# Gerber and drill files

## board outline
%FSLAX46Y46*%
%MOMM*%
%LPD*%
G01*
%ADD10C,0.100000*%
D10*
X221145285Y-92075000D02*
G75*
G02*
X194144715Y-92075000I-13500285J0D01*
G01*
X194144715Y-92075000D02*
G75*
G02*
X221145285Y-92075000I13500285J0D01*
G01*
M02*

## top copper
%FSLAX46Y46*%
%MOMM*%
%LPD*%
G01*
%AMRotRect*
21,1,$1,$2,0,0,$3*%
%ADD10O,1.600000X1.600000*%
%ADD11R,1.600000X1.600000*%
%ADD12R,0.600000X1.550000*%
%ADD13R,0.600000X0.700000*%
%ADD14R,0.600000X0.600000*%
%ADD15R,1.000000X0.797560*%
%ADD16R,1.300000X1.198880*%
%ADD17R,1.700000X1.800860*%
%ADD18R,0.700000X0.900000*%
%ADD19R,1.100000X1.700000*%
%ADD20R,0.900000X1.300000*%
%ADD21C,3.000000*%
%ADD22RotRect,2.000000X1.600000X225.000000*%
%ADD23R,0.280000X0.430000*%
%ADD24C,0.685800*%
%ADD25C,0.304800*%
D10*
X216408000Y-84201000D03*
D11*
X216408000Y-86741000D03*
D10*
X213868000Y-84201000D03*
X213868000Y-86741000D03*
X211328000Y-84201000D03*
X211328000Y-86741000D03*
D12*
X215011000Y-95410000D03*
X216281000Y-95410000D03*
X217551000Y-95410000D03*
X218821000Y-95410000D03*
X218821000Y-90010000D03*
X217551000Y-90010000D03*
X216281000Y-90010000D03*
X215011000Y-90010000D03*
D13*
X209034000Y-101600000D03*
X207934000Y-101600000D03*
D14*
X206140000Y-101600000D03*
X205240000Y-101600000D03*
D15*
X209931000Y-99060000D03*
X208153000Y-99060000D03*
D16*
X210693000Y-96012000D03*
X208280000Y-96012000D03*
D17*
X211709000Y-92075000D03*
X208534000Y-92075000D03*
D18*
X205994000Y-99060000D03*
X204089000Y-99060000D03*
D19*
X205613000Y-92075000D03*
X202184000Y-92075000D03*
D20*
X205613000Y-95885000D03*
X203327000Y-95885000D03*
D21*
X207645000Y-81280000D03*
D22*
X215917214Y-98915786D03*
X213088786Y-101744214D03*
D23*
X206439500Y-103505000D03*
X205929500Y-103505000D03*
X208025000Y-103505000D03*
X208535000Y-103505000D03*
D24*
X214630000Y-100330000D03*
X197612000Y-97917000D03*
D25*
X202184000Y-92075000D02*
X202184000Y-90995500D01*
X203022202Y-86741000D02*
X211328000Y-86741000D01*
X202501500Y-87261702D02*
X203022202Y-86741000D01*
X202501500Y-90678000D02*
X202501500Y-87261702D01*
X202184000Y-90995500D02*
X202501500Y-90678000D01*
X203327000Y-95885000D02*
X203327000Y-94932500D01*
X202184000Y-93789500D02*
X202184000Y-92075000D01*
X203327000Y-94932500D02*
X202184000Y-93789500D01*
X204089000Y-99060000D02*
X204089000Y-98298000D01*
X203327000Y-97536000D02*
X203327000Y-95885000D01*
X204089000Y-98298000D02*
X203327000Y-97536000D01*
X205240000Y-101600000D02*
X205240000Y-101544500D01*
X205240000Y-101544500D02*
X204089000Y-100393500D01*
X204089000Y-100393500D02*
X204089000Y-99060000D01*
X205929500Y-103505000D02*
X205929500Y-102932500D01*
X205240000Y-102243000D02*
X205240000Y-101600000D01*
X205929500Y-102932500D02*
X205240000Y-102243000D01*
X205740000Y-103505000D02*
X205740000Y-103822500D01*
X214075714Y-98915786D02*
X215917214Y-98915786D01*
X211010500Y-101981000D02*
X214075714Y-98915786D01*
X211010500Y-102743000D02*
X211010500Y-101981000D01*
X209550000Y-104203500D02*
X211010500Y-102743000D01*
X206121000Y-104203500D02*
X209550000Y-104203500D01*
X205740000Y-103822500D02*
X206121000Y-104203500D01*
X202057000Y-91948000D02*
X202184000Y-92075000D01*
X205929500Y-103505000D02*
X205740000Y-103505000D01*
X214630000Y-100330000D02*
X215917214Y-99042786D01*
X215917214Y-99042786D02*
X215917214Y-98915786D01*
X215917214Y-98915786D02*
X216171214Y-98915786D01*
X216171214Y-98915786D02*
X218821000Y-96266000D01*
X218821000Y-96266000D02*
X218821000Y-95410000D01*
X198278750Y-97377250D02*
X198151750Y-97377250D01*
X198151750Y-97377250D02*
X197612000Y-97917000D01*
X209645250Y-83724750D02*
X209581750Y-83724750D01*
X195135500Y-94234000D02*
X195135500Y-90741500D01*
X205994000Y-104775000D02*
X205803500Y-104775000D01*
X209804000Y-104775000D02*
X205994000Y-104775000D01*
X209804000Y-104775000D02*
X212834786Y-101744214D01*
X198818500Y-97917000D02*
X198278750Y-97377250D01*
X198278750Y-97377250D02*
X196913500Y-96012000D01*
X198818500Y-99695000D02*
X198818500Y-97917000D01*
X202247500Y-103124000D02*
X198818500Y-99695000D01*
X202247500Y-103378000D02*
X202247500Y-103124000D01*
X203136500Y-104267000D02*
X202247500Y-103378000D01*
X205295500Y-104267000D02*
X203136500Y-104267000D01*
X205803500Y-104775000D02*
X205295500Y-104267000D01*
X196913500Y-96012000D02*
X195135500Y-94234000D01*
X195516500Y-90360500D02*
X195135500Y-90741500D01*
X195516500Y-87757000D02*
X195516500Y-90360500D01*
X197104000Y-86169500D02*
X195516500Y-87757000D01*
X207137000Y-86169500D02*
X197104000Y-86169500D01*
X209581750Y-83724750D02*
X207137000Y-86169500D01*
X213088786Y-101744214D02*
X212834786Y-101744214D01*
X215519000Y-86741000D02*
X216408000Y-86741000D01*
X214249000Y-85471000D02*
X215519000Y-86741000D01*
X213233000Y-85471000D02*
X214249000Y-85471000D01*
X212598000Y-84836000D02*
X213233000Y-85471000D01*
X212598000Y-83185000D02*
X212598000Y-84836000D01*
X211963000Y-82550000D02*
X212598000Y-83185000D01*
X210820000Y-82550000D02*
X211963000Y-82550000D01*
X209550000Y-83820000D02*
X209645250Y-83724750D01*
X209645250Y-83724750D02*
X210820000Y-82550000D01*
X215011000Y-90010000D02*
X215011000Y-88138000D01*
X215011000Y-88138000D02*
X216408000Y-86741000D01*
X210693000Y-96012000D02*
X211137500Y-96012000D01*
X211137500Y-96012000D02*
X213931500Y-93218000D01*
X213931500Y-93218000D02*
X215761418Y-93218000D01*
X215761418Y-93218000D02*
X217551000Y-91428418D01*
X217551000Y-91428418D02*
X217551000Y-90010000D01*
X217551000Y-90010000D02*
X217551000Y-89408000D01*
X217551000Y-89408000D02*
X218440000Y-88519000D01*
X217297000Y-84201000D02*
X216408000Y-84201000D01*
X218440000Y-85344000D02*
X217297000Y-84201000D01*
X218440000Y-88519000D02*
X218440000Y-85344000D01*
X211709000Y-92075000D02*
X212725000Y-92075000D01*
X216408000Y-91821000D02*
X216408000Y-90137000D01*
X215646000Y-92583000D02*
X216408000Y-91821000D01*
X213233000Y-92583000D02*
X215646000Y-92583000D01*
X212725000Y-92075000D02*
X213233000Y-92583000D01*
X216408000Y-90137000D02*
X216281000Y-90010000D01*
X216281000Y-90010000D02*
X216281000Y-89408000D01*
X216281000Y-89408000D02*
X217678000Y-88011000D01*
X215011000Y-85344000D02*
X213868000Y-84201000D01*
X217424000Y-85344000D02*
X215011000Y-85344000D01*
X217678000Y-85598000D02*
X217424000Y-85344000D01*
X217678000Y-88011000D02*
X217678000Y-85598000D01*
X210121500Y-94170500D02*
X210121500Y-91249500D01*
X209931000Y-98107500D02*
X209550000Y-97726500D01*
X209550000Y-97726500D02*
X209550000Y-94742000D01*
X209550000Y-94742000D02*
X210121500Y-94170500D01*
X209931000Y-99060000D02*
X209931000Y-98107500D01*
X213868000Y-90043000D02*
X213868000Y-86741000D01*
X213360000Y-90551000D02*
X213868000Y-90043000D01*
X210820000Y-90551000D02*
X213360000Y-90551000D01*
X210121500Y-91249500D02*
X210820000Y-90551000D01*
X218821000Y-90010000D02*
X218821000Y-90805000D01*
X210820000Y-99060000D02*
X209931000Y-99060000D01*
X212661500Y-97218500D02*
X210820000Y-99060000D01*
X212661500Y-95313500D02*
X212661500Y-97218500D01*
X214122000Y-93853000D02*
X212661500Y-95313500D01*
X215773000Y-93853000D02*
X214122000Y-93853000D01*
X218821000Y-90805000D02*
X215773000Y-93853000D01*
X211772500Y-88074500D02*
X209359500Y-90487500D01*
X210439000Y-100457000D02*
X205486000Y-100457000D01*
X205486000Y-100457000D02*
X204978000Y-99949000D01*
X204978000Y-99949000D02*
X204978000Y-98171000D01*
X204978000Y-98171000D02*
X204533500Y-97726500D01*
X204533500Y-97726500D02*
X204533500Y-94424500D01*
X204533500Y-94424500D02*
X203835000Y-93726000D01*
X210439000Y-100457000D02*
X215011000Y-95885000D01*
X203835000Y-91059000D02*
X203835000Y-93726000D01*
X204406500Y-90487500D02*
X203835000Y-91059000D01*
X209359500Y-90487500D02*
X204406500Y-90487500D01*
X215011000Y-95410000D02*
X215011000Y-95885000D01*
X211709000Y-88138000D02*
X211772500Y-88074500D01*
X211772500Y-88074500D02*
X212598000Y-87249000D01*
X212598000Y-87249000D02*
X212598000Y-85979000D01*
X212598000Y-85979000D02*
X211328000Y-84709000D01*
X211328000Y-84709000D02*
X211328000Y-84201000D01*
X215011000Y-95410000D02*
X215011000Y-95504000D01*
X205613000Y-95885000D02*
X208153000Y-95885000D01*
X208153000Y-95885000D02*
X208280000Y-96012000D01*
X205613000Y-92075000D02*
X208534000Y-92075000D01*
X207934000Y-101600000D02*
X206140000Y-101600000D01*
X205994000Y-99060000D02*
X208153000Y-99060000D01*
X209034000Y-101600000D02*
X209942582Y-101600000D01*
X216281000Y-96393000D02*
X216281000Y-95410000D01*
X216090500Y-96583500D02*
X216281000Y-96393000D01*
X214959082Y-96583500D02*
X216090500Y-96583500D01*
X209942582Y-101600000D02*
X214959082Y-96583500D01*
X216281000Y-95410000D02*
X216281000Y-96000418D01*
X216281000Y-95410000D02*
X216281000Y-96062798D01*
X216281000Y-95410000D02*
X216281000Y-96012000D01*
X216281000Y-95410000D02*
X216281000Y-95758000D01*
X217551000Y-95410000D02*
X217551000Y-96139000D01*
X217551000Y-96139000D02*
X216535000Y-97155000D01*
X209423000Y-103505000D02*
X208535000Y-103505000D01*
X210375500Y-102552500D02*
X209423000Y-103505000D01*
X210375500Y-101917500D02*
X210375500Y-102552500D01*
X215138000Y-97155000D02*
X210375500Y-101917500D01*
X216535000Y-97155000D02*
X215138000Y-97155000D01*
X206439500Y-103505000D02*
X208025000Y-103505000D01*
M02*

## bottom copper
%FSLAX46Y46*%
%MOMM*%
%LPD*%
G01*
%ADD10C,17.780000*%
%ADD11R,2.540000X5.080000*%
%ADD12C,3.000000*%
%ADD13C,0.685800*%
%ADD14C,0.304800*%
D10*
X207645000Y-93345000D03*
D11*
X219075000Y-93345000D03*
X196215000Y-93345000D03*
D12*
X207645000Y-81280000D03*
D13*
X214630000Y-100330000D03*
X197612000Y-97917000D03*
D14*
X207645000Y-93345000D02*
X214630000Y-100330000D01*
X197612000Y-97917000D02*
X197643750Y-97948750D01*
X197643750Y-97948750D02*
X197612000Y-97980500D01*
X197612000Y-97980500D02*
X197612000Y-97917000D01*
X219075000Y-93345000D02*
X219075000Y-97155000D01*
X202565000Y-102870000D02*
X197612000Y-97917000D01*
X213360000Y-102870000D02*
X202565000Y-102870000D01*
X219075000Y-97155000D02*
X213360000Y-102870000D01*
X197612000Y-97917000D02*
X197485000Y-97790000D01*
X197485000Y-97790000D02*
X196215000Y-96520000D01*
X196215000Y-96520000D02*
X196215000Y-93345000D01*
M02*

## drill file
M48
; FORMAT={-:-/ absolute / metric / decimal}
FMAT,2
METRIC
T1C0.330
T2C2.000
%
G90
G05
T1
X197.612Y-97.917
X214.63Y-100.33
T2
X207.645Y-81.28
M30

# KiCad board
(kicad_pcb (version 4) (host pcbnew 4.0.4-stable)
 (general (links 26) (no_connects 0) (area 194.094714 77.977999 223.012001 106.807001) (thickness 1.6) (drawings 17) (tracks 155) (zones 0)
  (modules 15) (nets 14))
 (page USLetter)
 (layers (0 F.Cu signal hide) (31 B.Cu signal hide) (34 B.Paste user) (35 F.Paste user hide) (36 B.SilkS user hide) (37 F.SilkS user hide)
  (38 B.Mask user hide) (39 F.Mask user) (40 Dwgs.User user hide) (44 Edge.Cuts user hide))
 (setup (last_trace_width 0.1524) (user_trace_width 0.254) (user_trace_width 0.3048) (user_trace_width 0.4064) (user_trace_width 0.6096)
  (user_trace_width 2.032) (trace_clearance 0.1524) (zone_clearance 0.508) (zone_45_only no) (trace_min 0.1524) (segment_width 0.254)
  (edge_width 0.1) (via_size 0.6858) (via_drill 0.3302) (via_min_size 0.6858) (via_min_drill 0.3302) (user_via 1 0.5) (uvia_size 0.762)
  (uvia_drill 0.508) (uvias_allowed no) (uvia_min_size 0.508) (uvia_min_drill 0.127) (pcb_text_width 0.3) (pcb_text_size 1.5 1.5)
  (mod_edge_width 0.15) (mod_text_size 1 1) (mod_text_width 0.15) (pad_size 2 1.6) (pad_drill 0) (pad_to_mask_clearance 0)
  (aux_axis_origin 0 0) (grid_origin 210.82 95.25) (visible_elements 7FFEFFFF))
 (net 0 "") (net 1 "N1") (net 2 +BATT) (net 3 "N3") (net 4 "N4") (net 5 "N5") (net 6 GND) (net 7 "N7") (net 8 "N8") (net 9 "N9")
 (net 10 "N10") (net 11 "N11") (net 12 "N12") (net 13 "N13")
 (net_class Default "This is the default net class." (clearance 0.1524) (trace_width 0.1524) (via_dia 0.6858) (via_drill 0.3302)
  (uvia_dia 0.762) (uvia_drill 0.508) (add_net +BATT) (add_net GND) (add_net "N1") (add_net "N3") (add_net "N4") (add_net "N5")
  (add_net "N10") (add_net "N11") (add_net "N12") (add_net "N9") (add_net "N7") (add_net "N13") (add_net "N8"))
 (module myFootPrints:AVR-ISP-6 (layer F.Cu) (at 216.408 84.201 270)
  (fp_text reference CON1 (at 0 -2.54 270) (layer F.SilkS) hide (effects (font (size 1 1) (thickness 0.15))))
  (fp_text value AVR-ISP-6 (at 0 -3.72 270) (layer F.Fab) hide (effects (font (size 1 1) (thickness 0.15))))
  (pad 1 smd oval (at 0 0 270) (size 1.6 1.6) (layers F.Cu F.Paste F.Mask) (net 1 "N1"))
  (pad 2 smd rect (at 2.54 0 270) (size 1.6 1.6) (layers F.Cu F.Paste F.Mask) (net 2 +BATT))
  (pad 3 smd oval (at 0 2.54 270) (size 1.6 1.6) (layers F.Cu F.Paste F.Mask) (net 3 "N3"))
  (pad 4 smd oval (at 2.54 2.54 270) (size 1.6 1.6) (layers F.Cu F.Paste F.Mask) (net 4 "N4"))
  (pad 5 smd oval (at 0 5.08 270) (size 1.6 1.6) (layers F.Cu F.Paste F.Mask) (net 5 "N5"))
  (pad 6 smd oval (at 2.54 5.08 270) (size 1.6 1.6) (layers F.Cu F.Paste F.Mask) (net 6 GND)))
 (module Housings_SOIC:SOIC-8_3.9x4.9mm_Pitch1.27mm (layer F.Cu) (at 216.916 92.71 90)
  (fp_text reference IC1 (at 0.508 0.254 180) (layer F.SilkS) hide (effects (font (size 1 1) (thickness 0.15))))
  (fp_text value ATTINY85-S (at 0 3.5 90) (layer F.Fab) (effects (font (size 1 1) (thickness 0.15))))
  (pad 1 smd rect (at -2.7 -1.905 90) (size 1.55 0.6) (layers F.Cu F.Paste F.Mask) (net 5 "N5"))
  (pad 2 smd rect (at -2.7 -0.635 90) (size 1.55 0.6) (layers F.Cu F.Paste F.Mask) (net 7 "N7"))
  (pad 3 smd rect (at -2.7 0.635 90) (size 1.55 0.6) (layers F.Cu F.Paste F.Mask) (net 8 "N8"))
  (pad 4 smd rect (at -2.7 1.905 90) (size 1.55 0.6) (layers F.Cu F.Paste F.Mask) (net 6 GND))
  (pad 5 smd rect (at 2.7 1.905 90) (size 1.55 0.6) (layers F.Cu F.Paste F.Mask) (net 4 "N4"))
  (pad 6 smd rect (at 2.7 0.635 90) (size 1.55 0.6) (layers F.Cu F.Paste F.Mask) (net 1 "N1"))
  (pad 7 smd rect (at 2.7 -0.635 90) (size 1.55 0.6) (layers F.Cu F.Paste F.Mask) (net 3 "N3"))
  (pad 8 smd rect (at 2.7 -1.905 90) (size 1.55 0.6) (layers F.Cu F.Paste F.Mask) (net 2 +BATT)))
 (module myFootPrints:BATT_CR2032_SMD (layer B.Cu) (at 207.645 93.345 180)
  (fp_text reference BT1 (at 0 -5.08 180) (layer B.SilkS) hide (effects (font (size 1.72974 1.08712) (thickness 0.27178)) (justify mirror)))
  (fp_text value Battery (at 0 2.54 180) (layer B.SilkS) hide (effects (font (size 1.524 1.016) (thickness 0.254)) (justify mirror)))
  (pad 2 smd circle (at 0 0 180) (size 17.78 17.78) (layers B.Cu B.Paste B.Mask) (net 6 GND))
  (pad 1 smd rect (at -11.43 0 180) (size 2.54 5.08) (layers B.Cu B.Paste B.Mask) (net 2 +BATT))
  (pad 1 smd rect (at 11.43 0 180) (size 2.54 5.08) (layers B.Cu B.Paste B.Mask) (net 2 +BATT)))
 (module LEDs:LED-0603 (layer F.Cu) (at 208.534 101.6)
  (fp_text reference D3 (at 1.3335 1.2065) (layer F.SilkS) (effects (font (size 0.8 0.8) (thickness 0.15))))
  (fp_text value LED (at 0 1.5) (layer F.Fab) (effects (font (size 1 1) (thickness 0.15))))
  (pad 2 smd rect (at 0.5 0 180) (size 0.6 0.7) (layers F.Cu F.Paste F.Mask) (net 7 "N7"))
  (pad 1 smd rect (at -0.6 0 180) (size 0.6 0.7) (layers F.Cu F.Paste F.Mask) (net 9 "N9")))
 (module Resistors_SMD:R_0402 (layer F.Cu) (at 205.74 101.6 180)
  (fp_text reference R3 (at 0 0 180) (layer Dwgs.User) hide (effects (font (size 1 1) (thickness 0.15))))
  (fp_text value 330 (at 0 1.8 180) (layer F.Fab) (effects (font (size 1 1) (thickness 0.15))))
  (pad 1 smd rect (at -0.4 0 180) (size 0.6 0.6) (layers F.Cu F.Paste F.Mask) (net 9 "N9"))
  (pad 2 smd rect (at 0.5 0 180) (size 0.6 0.6) (layers F.Cu F.Paste F.Mask) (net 6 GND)))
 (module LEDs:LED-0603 (layer F.Cu) (at 209.042 99.06)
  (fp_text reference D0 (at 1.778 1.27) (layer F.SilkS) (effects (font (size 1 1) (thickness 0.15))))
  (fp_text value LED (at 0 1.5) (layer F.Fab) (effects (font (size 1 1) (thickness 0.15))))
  (pad 2 smd rect (at 0.889 0 180) (size 1 0.79756) (layers F.Cu F.Paste F.Mask) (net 4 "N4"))
  (pad 1 smd rect (at -0.889 0 180) (size 1 0.79756) (layers F.Cu F.Paste F.Mask) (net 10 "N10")))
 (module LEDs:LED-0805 (layer F.Cu) (at 209.55 96.012)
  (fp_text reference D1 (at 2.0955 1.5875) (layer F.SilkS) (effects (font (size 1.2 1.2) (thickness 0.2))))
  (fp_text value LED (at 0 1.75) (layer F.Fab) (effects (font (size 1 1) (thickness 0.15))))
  (pad 2 smd rect (at 1.143 0 180) (size 1.3 1.19888) (layers F.Cu F.Paste F.Mask) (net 1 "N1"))
  (pad 1 smd rect (at -1.27 0 180) (size 1.3 1.19888) (layers F.Cu F.Paste F.Mask) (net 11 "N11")))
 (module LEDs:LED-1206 (layer F.Cu) (at 210.185 92.075)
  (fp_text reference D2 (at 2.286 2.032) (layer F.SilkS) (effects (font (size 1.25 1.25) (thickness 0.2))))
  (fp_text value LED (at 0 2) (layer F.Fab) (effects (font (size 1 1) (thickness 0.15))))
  (pad 2 smd rect (at 1.524 0 180) (size 1.7 1.80086) (layers F.Cu F.Paste F.Mask) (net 3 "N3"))
  (pad 1 smd rect (at -1.651 0 180) (size 1.7 1.80086) (layers F.Cu F.Paste F.Mask) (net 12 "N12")))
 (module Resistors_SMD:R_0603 (layer F.Cu) (at 205.105 99.06 180)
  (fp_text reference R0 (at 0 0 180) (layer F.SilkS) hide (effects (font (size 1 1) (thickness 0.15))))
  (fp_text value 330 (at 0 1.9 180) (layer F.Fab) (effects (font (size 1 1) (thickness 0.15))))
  (pad 1 smd rect (at -0.889 0 180) (size 0.7 0.9) (layers F.Cu F.Paste F.Mask) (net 10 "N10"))
  (pad 2 smd rect (at 1.016 0 180) (size 0.7 0.9) (layers F.Cu F.Paste F.Mask) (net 6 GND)))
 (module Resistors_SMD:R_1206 (layer F.Cu) (at 203.835 92.075 180)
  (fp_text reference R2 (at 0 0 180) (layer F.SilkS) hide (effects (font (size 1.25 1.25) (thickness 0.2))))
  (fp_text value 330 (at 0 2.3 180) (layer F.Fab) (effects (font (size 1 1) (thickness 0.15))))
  (pad 1 smd rect (at -1.778 0 180) (size 1.1 1.7) (layers F.Cu F.Paste F.Mask) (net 12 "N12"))
  (pad 2 smd rect (at 1.651 0 180) (size 1.1 1.7) (layers F.Cu F.Paste F.Mask) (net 6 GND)))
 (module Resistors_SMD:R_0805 (layer F.Cu) (at 204.47 95.885 180)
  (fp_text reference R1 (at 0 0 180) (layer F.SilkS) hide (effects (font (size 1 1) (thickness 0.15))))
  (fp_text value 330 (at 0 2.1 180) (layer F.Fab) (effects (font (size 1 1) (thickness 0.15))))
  (pad 1 smd rect (at -1.143 0 180) (size 0.9 1.3) (layers F.Cu F.Paste F.Mask) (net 11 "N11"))
  (pad 2 smd rect (at 1.143 0 180) (size 0.9 1.3) (layers F.Cu F.Paste F.Mask) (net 6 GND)))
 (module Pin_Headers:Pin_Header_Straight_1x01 (layer F.Cu) (at 207.645 81.28)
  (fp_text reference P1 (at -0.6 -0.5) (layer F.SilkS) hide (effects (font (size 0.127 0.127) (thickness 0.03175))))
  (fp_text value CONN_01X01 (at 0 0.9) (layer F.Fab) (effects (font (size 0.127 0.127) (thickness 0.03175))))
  (pad "" thru_hole circle (at 0 0) (size 3 3) (drill 2) (layers *.Cu *.Mask)))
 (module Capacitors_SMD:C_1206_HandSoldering (layer F.Cu) (at 214.503 100.33 225)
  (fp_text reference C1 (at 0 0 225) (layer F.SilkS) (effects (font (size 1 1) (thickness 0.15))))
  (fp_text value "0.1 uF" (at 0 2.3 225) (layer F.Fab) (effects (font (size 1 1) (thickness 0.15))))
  (pad 1 smd rect (at -2 0 225) (size 2 1.6) (layers F.Cu F.Paste F.Mask) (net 6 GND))
  (pad 2 smd rect (at 2 0 225) (size 2 1.6) (layers F.Cu F.Paste F.Mask) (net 2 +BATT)))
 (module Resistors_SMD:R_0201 (layer F.Cu) (at 206.1845 103.505 180)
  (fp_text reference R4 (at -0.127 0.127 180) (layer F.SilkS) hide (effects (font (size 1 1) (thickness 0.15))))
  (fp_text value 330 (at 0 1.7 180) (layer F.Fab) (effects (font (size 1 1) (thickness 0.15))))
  (pad 1 smd rect (at -0.255 0 180) (size 0.28 0.43) (layers F.Cu F.Paste F.Mask) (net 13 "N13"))
  (pad 2 smd rect (at 0.255 0 180) (size 0.28 0.43) (layers F.Cu F.Paste F.Mask) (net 6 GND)))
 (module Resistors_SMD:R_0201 (layer F.Cu) (at 208.28 103.505)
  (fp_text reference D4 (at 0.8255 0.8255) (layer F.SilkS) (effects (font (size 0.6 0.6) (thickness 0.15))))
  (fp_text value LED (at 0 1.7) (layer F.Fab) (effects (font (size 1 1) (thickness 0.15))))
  (pad 1 smd rect (at -0.255 0) (size 0.28 0.43) (layers F.Cu F.Paste F.Mask) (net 13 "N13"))
  (pad 2 smd rect (at 0.255 0) (size 0.28 0.43) (layers F.Cu F.Paste F.Mask) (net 8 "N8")))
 (gr_circle (center 207.645 92.075) (end 197.485 83.185) (layer Edge.Cuts) (width 0.1))
 (segment (start 202.184 92.075) (end 202.184 90.9955) (width 0.3048) (layer F.Cu) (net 6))
 (segment (start 203.022202 86.741) (end 211.328 86.741) (width 0.3048) (layer F.Cu) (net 6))
 (segment (start 202.5015 87.261702) (end 203.022202 86.741) (width 0.3048) (layer F.Cu) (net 6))
 (segment (start 202.5015 90.678) (end 202.5015 87.261702) (width 0.3048) (layer F.Cu) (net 6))
 (segment (start 202.184 90.9955) (end 202.5015 90.678) (width 0.3048) (layer F.Cu) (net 6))
 (segment (start 203.327 95.885) (end 203.327 94.9325) (width 0.3048) (layer F.Cu) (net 6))
 (segment (start 202.184 93.7895) (end 202.184 92.075) (width 0.3048) (layer F.Cu) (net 6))
 (segment (start 203.327 94.9325) (end 202.184 93.7895) (width 0.3048) (layer F.Cu) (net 6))
 (segment (start 204.089 99.06) (end 204.089 98.298) (width 0.3048) (layer F.Cu) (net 6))
 (segment (start 203.327 97.536) (end 203.327 95.885) (width 0.3048) (layer F.Cu) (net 6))
 (segment (start 204.089 98.298) (end 203.327 97.536) (width 0.3048) (layer F.Cu) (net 6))
 (segment (start 205.24 101.6) (end 205.24 101.5445) (width 0.3048) (layer F.Cu) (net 6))
 (segment (start 205.24 101.5445) (end 204.089 100.3935) (width 0.3048) (layer F.Cu) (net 6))
 (segment (start 204.089 100.3935) (end 204.089 99.06) (width 0.3048) (layer F.Cu) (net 6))
 (segment (start 205.9295 103.505) (end 205.9295 102.9325) (width 0.3048) (layer F.Cu) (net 6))
 (segment (start 205.24 102.243) (end 205.24 101.6) (width 0.3048) (layer F.Cu) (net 6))
 (segment (start 205.9295 102.9325) (end 205.24 102.243) (width 0.3048) (layer F.Cu) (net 6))
 (segment (start 205.74 103.505) (end 205.74 103.8225) (width 0.3048) (layer F.Cu) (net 6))
 (segment (start 214.075714 98.915786) (end 215.917214 98.915786) (width 0.3048) (layer F.Cu) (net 6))
 (segment (start 211.0105 101.981) (end 214.075714 98.915786) (width 0.3048) (layer F.Cu) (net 6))
 (segment (start 211.0105 102.743) (end 211.0105 101.981) (width 0.3048) (layer F.Cu) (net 6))
 (segment (start 209.55 104.2035) (end 211.0105 102.743) (width 0.3048) (layer F.Cu) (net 6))
 (segment (start 206.121 104.2035) (end 209.55 104.2035) (width 0.3048) (layer F.Cu) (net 6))
 (segment (start 205.74 103.8225) (end 206.121 104.2035) (width 0.3048) (layer F.Cu) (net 6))
 (segment (start 202.057 91.948) (end 202.184 92.075) (width 0.3048) (layer F.Cu) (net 6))
 (segment (start 205.9295 103.505) (end 205.74 103.505) (width 0.3048) (layer F.Cu) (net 6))
 (segment (start 207.645 93.345) (end 214.63 100.33) (width 0.3048) (layer B.Cu) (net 6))
 (segment (start 214.63 100.33) (end 215.917214 99.042786) (width 0.3048) (layer F.Cu) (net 6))
 (via (at 214.63 100.33) (size 0.6858) (drill 0.3302) (layers F.Cu B.Cu) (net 6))
 (segment (start 215.917214 99.042786) (end 215.917214 98.915786) (width 0.3048) (layer F.Cu) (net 6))
 (segment (start 215.917214 98.915786) (end 216.171214 98.915786) (width 0.3048) (layer F.Cu) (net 6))
 (segment (start 216.171214 98.915786) (end 218.821 96.266) (width 0.3048) (layer F.Cu) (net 6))
 (segment (start 218.821 96.266) (end 218.821 95.41) (width 0.3048) (layer F.Cu) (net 6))
 (segment (start 198.27875 97.37725) (end 198.15175 97.37725) (width 0.3048) (layer F.Cu) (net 2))
 (via (at 197.612 97.917) (size 0.6858) (drill 0.3302) (layers F.Cu B.Cu) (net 2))
 (segment (start 198.15175 97.37725) (end 197.612 97.917) (width 0.3048) (layer F.Cu) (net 2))
 (segment (start 197.612 97.917) (end 197.64375 97.94875) (width 0.3048) (layer B.Cu) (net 2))
 (segment (start 197.64375 97.94875) (end 197.612 97.9805) (width 0.3048) (layer B.Cu) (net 2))
 (segment (start 197.612 97.9805) (end 197.612 97.917) (width 0.3048) (layer B.Cu) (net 2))
 (segment (start 209.64525 83.72475) (end 209.58175 83.72475) (width 0.3048) (layer F.Cu) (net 2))
 (segment (start 195.1355 94.234) (end 195.1355 90.7415) (width 0.3048) (layer F.Cu) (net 2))
 (segment (start 205.994 104.775) (end 205.8035 104.775) (width 0.3048) (layer F.Cu) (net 2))
 (segment (start 209.804 104.775) (end 205.994 104.775) (width 0.3048) (layer F.Cu) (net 2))
 (segment (start 209.804 104.775) (end 212.834786 101.744214) (width 0.3048) (layer F.Cu) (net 2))
 (segment (start 198.8185 97.917) (end 198.27875 97.37725) (width 0.3048) (layer F.Cu) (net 2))
 (segment (start 198.27875 97.37725) (end 196.9135 96.012) (width 0.3048) (layer F.Cu) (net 2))
 (segment (start 198.8185 99.695) (end 198.8185 97.917) (width 0.3048) (layer F.Cu) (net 2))
 (segment (start 202.2475 103.124) (end 198.8185 99.695) (width 0.3048) (layer F.Cu) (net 2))
 (segment (start 202.2475 103.378) (end 202.2475 103.124) (width 0.3048) (layer F.Cu) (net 2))
 (segment (start 203.1365 104.267) (end 202.2475 103.378) (width 0.3048) (layer F.Cu) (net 2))
 (segment (start 205.2955 104.267) (end 203.1365 104.267) (width 0.3048) (layer F.Cu) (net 2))
 (segment (start 205.8035 104.775) (end 205.2955 104.267) (width 0.3048) (layer F.Cu) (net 2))
 (segment (start 196.9135 96.012) (end 195.1355 94.234) (width 0.3048) (layer F.Cu) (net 2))
 (segment (start 195.5165 90.3605) (end 195.1355 90.7415) (width 0.3048) (layer F.Cu) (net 2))
 (segment (start 195.5165 87.757) (end 195.5165 90.3605) (width 0.3048) (layer F.Cu) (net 2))
 (segment (start 197.104 86.1695) (end 195.5165 87.757) (width 0.3048) (layer F.Cu) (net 2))
 (segment (start 207.137 86.1695) (end 197.104 86.1695) (width 0.3048) (layer F.Cu) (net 2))
 (segment (start 209.58175 83.72475) (end 207.137 86.1695) (width 0.3048) (layer F.Cu) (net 2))
 (segment (start 219.075 93.345) (end 219.075 97.155) (width 0.3048) (layer B.Cu) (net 2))
 (segment (start 202.565 102.87) (end 197.612 97.917) (width 0.3048) (layer B.Cu) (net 2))
 (segment (start 213.36 102.87) (end 202.565 102.87) (width 0.3048) (layer B.Cu) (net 2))
 (segment (start 219.075 97.155) (end 213.36 102.87) (width 0.3048) (layer B.Cu) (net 2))
 (segment (start 197.612 97.917) (end 197.485 97.79) (width 0.3048) (layer B.Cu) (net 2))
 (segment (start 197.485 97.79) (end 196.215 96.52) (width 0.3048) (layer B.Cu) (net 2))
 (segment (start 196.215 96.52) (end 196.215 93.345) (width 0.3048) (layer B.Cu) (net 2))
 (segment (start 213.088786 101.744214) (end 212.834786 101.744214) (width 0.3048) (layer F.Cu) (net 2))
 (segment (start 215.519 86.741) (end 216.408 86.741) (width 0.3048) (layer F.Cu) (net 2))
 (segment (start 214.249 85.471) (end 215.519 86.741) (width 0.3048) (layer F.Cu) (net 2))
 (segment (start 213.233 85.471) (end 214.249 85.471) (width 0.3048) (layer F.Cu) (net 2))
 (segment (start 212.598 84.836) (end 213.233 85.471) (width 0.3048) (layer F.Cu) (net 2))
 (segment (start 212.598 83.185) (end 212.598 84.836) (width 0.3048) (layer F.Cu) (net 2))
 (segment (start 211.963 82.55) (end 212.598 83.185) (width 0.3048) (layer F.Cu) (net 2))
 (segment (start 210.82 82.55) (end 211.963 82.55) (width 0.3048) (layer F.Cu) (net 2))
 (segment (start 209.55 83.82) (end 209.64525 83.72475) (width 0.3048) (layer F.Cu) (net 2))
 (segment (start 209.64525 83.72475) (end 210.82 82.55) (width 0.3048) (layer F.Cu) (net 2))
 (segment (start 215.011 90.01) (end 215.011 88.138) (width 0.3048) (layer F.Cu) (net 2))
 (segment (start 215.011 88.138) (end 216.408 86.741) (width 0.3048) (layer F.Cu) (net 2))
 (segment (start 210.693 96.012) (end 211.1375 96.012) (width 0.3048) (layer F.Cu) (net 1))
 (segment (start 211.1375 96.012) (end 213.9315 93.218) (width 0.3048) (layer F.Cu) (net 1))
 (segment (start 213.9315 93.218) (end 215.761418 93.218) (width 0.3048) (layer F.Cu) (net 1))
 (segment (start 215.761418 93.218) (end 217.551 91.428418) (width 0.3048) (layer F.Cu) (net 1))
 (segment (start 217.551 91.428418) (end 217.551 90.01) (width 0.3048) (layer F.Cu) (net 1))
 (segment (start 217.551 90.01) (end 217.551 89.408) (width 0.3048) (layer F.Cu) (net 1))
 (segment (start 217.551 89.408) (end 218.44 88.519) (width 0.3048) (layer F.Cu) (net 1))
 (segment (start 217.297 84.201) (end 216.408 84.201) (width 0.3048) (layer F.Cu) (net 1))
 (segment (start 218.44 85.344) (end 217.297 84.201) (width 0.3048) (layer F.Cu) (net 1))
 (segment (start 218.44 88.519) (end 218.44 85.344) (width 0.3048) (layer F.Cu) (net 1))
 (segment (start 211.709 92.075) (end 212.725 92.075) (width 0.3048) (layer F.Cu) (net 3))
 (segment (start 216.408 91.821) (end 216.408 90.137) (width 0.3048) (layer F.Cu) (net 3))
 (segment (start 215.646 92.583) (end 216.408 91.821) (width 0.3048) (layer F.Cu) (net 3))
 (segment (start 213.233 92.583) (end 215.646 92.583) (width 0.3048) (layer F.Cu) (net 3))
 (segment (start 212.725 92.075) (end 213.233 92.583) (width 0.3048) (layer F.Cu) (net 3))
 (segment (start 216.408 90.137) (end 216.281 90.01) (width 0.3048) (layer F.Cu) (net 3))
 (segment (start 216.281 90.01) (end 216.281 89.408) (width 0.3048) (layer F.Cu) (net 3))
 (segment (start 216.281 89.408) (end 217.678 88.011) (width 0.3048) (layer F.Cu) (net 3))
 (segment (start 215.011 85.344) (end 213.868 84.201) (width 0.3048) (layer F.Cu) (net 3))
 (segment (start 217.424 85.344) (end 215.011 85.344) (width 0.3048) (layer F.Cu) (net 3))
 (segment (start 217.678 85.598) (end 217.424 85.344) (width 0.3048) (layer F.Cu) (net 3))
 (segment (start 217.678 88.011) (end 217.678 85.598) (width 0.3048) (layer F.Cu) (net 3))
 (segment (start 210.1215 94.1705) (end 210.1215 91.2495) (width 0.3048) (layer F.Cu) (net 4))
 (segment (start 209.931 98.1075) (end 209.55 97.7265) (width 0.3048) (layer F.Cu) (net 4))
 (segment (start 209.55 97.7265) (end 209.55 94.742) (width 0.3048) (layer F.Cu) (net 4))
 (segment (start 209.55 94.742) (end 210.1215 94.1705) (width 0.3048) (layer F.Cu) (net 4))
 (segment (start 209.931 99.06) (end 209.931 98.1075) (width 0.3048) (layer F.Cu) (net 4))
 (segment (start 213.868 90.043) (end 213.868 86.741) (width 0.3048) (layer F.Cu) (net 4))
 (segment (start 213.36 90.551) (end 213.868 90.043) (width 0.3048) (layer F.Cu) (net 4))
 (segment (start 210.82 90.551) (end 213.36 90.551) (width 0.3048) (layer F.Cu) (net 4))
 (segment (start 210.1215 91.2495) (end 210.82 90.551) (width 0.3048) (layer F.Cu) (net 4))
 (segment (start 218.821 90.01) (end 218.821 90.805) (width 0.3048) (layer F.Cu) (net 4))
 (segment (start 210.82 99.06) (end 209.931 99.06) (width 0.3048) (layer F.Cu) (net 4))
 (segment (start 212.6615 97.2185) (end 210.82 99.06) (width 0.3048) (layer F.Cu) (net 4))
 (segment (start 212.6615 95.3135) (end 212.6615 97.2185) (width 0.3048) (layer F.Cu) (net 4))
 (segment (start 214.122 93.853) (end 212.6615 95.3135) (width 0.3048) (layer F.Cu) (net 4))
 (segment (start 215.773 93.853) (end 214.122 93.853) (width 0.3048) (layer F.Cu) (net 4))
 (segment (start 218.821 90.805) (end 215.773 93.853) (width 0.3048) (layer F.Cu) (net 4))
 (segment (start 211.7725 88.0745) (end 209.3595 90.4875) (width 0.3048) (layer F.Cu) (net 5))
 (segment (start 210.439 100.457) (end 205.486 100.457) (width 0.3048) (layer F.Cu) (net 5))
 (segment (start 205.486 100.457) (end 204.978 99.949) (width 0.3048) (layer F.Cu) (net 5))
 (segment (start 204.978 99.949) (end 204.978 98.171) (width 0.3048) (layer F.Cu) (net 5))
 (segment (start 204.978 98.171) (end 204.5335 97.7265) (width 0.3048) (layer F.Cu) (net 5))
 (segment (start 204.5335 97.7265) (end 204.5335 94.4245) (width 0.3048) (layer F.Cu) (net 5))
 (segment (start 204.5335 94.4245) (end 203.835 93.726) (width 0.3048) (layer F.Cu) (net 5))
 (segment (start 210.439 100.457) (end 215.011 95.885) (width 0.3048) (layer F.Cu) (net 5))
 (segment (start 203.835 91.059) (end 203.835 93.726) (width 0.3048) (layer F.Cu) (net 5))
 (segment (start 204.4065 90.4875) (end 203.835 91.059) (width 0.3048) (layer F.Cu) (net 5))
 (segment (start 209.3595 90.4875) (end 204.4065 90.4875) (width 0.3048) (layer F.Cu) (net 5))
 (segment (start 215.011 95.41) (end 215.011 95.885) (width 0.3048) (layer F.Cu) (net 5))
 (segment (start 211.709 88.138) (end 211.7725 88.0745) (width 0.3048) (layer F.Cu) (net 5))
 (segment (start 211.7725 88.0745) (end 212.598 87.249) (width 0.3048) (layer F.Cu) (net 5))
 (segment (start 212.598 87.249) (end 212.598 85.979) (width 0.3048) (layer F.Cu) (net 5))
 (segment (start 212.598 85.979) (end 211.328 84.709) (width 0.3048) (layer F.Cu) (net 5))
 (segment (start 211.328 84.709) (end 211.328 84.201) (width 0.3048) (layer F.Cu) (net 5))
 (segment (start 215.011 95.41) (end 215.011 95.504) (width 0.3048) (layer F.Cu) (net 5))
 (segment (start 205.613 95.885) (end 208.153 95.885) (width 0.3048) (layer F.Cu) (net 11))
 (segment (start 208.153 95.885) (end 208.28 96.012) (width 0.3048) (layer F.Cu) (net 11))
 (segment (start 205.613 92.075) (end 208.534 92.075) (width 0.3048) (layer F.Cu) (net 12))
 (segment (start 207.934 101.6) (end 206.14 101.6) (width 0.3048) (layer F.Cu) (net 9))
 (segment (start 205.994 99.06) (end 208.153 99.06) (width 0.3048) (layer F.Cu) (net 10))
 (segment (start 209.034 101.6) (end 209.942582 101.6) (width 0.3048) (layer F.Cu) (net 7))
 (segment (start 216.281 96.393) (end 216.281 95.41) (width 0.3048) (layer F.Cu) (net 7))
 (segment (start 216.0905 96.5835) (end 216.281 96.393) (width 0.3048) (layer F.Cu) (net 7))
 (segment (start 214.959082 96.5835) (end 216.0905 96.5835) (width 0.3048) (layer F.Cu) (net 7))
 (segment (start 209.942582 101.6) (end 214.959082 96.5835) (width 0.3048) (layer F.Cu) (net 7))
 (segment (start 216.281 95.41) (end 216.281 96.000418) (width 0.3048) (layer F.Cu) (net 7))
 (segment (start 216.281 95.41) (end 216.281 96.062798) (width 0.3048) (layer F.Cu) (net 7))
 (segment (start 216.281 95.41) (end 216.281 96.012) (width 0.3048) (layer F.Cu) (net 7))
 (segment (start 216.281 95.41) (end 216.281 95.758) (width 0.3048) (layer F.Cu) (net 7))
 (segment (start 217.551 95.41) (end 217.551 96.139) (width 0.3048) (layer F.Cu) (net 8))
 (segment (start 217.551 96.139) (end 216.535 97.155) (width 0.3048) (layer F.Cu) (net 8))
 (segment (start 209.423 103.505) (end 208.535 103.505) (width 0.3048) (layer F.Cu) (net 8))
 (segment (start 210.3755 102.5525) (end 209.423 103.505) (width 0.3048) (layer F.Cu) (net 8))
 (segment (start 210.3755 101.9175) (end 210.3755 102.5525) (width 0.3048) (layer F.Cu) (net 8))
 (segment (start 215.138 97.155) (end 210.3755 101.9175) (width 0.3048) (layer F.Cu) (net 8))
 (segment (start 216.535 97.155) (end 215.138 97.155) (width 0.3048) (layer F.Cu) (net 8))
 (segment (start 206.4395 103.505) (end 208.025 103.505) (width 0.3048) (layer F.Cu) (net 13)))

